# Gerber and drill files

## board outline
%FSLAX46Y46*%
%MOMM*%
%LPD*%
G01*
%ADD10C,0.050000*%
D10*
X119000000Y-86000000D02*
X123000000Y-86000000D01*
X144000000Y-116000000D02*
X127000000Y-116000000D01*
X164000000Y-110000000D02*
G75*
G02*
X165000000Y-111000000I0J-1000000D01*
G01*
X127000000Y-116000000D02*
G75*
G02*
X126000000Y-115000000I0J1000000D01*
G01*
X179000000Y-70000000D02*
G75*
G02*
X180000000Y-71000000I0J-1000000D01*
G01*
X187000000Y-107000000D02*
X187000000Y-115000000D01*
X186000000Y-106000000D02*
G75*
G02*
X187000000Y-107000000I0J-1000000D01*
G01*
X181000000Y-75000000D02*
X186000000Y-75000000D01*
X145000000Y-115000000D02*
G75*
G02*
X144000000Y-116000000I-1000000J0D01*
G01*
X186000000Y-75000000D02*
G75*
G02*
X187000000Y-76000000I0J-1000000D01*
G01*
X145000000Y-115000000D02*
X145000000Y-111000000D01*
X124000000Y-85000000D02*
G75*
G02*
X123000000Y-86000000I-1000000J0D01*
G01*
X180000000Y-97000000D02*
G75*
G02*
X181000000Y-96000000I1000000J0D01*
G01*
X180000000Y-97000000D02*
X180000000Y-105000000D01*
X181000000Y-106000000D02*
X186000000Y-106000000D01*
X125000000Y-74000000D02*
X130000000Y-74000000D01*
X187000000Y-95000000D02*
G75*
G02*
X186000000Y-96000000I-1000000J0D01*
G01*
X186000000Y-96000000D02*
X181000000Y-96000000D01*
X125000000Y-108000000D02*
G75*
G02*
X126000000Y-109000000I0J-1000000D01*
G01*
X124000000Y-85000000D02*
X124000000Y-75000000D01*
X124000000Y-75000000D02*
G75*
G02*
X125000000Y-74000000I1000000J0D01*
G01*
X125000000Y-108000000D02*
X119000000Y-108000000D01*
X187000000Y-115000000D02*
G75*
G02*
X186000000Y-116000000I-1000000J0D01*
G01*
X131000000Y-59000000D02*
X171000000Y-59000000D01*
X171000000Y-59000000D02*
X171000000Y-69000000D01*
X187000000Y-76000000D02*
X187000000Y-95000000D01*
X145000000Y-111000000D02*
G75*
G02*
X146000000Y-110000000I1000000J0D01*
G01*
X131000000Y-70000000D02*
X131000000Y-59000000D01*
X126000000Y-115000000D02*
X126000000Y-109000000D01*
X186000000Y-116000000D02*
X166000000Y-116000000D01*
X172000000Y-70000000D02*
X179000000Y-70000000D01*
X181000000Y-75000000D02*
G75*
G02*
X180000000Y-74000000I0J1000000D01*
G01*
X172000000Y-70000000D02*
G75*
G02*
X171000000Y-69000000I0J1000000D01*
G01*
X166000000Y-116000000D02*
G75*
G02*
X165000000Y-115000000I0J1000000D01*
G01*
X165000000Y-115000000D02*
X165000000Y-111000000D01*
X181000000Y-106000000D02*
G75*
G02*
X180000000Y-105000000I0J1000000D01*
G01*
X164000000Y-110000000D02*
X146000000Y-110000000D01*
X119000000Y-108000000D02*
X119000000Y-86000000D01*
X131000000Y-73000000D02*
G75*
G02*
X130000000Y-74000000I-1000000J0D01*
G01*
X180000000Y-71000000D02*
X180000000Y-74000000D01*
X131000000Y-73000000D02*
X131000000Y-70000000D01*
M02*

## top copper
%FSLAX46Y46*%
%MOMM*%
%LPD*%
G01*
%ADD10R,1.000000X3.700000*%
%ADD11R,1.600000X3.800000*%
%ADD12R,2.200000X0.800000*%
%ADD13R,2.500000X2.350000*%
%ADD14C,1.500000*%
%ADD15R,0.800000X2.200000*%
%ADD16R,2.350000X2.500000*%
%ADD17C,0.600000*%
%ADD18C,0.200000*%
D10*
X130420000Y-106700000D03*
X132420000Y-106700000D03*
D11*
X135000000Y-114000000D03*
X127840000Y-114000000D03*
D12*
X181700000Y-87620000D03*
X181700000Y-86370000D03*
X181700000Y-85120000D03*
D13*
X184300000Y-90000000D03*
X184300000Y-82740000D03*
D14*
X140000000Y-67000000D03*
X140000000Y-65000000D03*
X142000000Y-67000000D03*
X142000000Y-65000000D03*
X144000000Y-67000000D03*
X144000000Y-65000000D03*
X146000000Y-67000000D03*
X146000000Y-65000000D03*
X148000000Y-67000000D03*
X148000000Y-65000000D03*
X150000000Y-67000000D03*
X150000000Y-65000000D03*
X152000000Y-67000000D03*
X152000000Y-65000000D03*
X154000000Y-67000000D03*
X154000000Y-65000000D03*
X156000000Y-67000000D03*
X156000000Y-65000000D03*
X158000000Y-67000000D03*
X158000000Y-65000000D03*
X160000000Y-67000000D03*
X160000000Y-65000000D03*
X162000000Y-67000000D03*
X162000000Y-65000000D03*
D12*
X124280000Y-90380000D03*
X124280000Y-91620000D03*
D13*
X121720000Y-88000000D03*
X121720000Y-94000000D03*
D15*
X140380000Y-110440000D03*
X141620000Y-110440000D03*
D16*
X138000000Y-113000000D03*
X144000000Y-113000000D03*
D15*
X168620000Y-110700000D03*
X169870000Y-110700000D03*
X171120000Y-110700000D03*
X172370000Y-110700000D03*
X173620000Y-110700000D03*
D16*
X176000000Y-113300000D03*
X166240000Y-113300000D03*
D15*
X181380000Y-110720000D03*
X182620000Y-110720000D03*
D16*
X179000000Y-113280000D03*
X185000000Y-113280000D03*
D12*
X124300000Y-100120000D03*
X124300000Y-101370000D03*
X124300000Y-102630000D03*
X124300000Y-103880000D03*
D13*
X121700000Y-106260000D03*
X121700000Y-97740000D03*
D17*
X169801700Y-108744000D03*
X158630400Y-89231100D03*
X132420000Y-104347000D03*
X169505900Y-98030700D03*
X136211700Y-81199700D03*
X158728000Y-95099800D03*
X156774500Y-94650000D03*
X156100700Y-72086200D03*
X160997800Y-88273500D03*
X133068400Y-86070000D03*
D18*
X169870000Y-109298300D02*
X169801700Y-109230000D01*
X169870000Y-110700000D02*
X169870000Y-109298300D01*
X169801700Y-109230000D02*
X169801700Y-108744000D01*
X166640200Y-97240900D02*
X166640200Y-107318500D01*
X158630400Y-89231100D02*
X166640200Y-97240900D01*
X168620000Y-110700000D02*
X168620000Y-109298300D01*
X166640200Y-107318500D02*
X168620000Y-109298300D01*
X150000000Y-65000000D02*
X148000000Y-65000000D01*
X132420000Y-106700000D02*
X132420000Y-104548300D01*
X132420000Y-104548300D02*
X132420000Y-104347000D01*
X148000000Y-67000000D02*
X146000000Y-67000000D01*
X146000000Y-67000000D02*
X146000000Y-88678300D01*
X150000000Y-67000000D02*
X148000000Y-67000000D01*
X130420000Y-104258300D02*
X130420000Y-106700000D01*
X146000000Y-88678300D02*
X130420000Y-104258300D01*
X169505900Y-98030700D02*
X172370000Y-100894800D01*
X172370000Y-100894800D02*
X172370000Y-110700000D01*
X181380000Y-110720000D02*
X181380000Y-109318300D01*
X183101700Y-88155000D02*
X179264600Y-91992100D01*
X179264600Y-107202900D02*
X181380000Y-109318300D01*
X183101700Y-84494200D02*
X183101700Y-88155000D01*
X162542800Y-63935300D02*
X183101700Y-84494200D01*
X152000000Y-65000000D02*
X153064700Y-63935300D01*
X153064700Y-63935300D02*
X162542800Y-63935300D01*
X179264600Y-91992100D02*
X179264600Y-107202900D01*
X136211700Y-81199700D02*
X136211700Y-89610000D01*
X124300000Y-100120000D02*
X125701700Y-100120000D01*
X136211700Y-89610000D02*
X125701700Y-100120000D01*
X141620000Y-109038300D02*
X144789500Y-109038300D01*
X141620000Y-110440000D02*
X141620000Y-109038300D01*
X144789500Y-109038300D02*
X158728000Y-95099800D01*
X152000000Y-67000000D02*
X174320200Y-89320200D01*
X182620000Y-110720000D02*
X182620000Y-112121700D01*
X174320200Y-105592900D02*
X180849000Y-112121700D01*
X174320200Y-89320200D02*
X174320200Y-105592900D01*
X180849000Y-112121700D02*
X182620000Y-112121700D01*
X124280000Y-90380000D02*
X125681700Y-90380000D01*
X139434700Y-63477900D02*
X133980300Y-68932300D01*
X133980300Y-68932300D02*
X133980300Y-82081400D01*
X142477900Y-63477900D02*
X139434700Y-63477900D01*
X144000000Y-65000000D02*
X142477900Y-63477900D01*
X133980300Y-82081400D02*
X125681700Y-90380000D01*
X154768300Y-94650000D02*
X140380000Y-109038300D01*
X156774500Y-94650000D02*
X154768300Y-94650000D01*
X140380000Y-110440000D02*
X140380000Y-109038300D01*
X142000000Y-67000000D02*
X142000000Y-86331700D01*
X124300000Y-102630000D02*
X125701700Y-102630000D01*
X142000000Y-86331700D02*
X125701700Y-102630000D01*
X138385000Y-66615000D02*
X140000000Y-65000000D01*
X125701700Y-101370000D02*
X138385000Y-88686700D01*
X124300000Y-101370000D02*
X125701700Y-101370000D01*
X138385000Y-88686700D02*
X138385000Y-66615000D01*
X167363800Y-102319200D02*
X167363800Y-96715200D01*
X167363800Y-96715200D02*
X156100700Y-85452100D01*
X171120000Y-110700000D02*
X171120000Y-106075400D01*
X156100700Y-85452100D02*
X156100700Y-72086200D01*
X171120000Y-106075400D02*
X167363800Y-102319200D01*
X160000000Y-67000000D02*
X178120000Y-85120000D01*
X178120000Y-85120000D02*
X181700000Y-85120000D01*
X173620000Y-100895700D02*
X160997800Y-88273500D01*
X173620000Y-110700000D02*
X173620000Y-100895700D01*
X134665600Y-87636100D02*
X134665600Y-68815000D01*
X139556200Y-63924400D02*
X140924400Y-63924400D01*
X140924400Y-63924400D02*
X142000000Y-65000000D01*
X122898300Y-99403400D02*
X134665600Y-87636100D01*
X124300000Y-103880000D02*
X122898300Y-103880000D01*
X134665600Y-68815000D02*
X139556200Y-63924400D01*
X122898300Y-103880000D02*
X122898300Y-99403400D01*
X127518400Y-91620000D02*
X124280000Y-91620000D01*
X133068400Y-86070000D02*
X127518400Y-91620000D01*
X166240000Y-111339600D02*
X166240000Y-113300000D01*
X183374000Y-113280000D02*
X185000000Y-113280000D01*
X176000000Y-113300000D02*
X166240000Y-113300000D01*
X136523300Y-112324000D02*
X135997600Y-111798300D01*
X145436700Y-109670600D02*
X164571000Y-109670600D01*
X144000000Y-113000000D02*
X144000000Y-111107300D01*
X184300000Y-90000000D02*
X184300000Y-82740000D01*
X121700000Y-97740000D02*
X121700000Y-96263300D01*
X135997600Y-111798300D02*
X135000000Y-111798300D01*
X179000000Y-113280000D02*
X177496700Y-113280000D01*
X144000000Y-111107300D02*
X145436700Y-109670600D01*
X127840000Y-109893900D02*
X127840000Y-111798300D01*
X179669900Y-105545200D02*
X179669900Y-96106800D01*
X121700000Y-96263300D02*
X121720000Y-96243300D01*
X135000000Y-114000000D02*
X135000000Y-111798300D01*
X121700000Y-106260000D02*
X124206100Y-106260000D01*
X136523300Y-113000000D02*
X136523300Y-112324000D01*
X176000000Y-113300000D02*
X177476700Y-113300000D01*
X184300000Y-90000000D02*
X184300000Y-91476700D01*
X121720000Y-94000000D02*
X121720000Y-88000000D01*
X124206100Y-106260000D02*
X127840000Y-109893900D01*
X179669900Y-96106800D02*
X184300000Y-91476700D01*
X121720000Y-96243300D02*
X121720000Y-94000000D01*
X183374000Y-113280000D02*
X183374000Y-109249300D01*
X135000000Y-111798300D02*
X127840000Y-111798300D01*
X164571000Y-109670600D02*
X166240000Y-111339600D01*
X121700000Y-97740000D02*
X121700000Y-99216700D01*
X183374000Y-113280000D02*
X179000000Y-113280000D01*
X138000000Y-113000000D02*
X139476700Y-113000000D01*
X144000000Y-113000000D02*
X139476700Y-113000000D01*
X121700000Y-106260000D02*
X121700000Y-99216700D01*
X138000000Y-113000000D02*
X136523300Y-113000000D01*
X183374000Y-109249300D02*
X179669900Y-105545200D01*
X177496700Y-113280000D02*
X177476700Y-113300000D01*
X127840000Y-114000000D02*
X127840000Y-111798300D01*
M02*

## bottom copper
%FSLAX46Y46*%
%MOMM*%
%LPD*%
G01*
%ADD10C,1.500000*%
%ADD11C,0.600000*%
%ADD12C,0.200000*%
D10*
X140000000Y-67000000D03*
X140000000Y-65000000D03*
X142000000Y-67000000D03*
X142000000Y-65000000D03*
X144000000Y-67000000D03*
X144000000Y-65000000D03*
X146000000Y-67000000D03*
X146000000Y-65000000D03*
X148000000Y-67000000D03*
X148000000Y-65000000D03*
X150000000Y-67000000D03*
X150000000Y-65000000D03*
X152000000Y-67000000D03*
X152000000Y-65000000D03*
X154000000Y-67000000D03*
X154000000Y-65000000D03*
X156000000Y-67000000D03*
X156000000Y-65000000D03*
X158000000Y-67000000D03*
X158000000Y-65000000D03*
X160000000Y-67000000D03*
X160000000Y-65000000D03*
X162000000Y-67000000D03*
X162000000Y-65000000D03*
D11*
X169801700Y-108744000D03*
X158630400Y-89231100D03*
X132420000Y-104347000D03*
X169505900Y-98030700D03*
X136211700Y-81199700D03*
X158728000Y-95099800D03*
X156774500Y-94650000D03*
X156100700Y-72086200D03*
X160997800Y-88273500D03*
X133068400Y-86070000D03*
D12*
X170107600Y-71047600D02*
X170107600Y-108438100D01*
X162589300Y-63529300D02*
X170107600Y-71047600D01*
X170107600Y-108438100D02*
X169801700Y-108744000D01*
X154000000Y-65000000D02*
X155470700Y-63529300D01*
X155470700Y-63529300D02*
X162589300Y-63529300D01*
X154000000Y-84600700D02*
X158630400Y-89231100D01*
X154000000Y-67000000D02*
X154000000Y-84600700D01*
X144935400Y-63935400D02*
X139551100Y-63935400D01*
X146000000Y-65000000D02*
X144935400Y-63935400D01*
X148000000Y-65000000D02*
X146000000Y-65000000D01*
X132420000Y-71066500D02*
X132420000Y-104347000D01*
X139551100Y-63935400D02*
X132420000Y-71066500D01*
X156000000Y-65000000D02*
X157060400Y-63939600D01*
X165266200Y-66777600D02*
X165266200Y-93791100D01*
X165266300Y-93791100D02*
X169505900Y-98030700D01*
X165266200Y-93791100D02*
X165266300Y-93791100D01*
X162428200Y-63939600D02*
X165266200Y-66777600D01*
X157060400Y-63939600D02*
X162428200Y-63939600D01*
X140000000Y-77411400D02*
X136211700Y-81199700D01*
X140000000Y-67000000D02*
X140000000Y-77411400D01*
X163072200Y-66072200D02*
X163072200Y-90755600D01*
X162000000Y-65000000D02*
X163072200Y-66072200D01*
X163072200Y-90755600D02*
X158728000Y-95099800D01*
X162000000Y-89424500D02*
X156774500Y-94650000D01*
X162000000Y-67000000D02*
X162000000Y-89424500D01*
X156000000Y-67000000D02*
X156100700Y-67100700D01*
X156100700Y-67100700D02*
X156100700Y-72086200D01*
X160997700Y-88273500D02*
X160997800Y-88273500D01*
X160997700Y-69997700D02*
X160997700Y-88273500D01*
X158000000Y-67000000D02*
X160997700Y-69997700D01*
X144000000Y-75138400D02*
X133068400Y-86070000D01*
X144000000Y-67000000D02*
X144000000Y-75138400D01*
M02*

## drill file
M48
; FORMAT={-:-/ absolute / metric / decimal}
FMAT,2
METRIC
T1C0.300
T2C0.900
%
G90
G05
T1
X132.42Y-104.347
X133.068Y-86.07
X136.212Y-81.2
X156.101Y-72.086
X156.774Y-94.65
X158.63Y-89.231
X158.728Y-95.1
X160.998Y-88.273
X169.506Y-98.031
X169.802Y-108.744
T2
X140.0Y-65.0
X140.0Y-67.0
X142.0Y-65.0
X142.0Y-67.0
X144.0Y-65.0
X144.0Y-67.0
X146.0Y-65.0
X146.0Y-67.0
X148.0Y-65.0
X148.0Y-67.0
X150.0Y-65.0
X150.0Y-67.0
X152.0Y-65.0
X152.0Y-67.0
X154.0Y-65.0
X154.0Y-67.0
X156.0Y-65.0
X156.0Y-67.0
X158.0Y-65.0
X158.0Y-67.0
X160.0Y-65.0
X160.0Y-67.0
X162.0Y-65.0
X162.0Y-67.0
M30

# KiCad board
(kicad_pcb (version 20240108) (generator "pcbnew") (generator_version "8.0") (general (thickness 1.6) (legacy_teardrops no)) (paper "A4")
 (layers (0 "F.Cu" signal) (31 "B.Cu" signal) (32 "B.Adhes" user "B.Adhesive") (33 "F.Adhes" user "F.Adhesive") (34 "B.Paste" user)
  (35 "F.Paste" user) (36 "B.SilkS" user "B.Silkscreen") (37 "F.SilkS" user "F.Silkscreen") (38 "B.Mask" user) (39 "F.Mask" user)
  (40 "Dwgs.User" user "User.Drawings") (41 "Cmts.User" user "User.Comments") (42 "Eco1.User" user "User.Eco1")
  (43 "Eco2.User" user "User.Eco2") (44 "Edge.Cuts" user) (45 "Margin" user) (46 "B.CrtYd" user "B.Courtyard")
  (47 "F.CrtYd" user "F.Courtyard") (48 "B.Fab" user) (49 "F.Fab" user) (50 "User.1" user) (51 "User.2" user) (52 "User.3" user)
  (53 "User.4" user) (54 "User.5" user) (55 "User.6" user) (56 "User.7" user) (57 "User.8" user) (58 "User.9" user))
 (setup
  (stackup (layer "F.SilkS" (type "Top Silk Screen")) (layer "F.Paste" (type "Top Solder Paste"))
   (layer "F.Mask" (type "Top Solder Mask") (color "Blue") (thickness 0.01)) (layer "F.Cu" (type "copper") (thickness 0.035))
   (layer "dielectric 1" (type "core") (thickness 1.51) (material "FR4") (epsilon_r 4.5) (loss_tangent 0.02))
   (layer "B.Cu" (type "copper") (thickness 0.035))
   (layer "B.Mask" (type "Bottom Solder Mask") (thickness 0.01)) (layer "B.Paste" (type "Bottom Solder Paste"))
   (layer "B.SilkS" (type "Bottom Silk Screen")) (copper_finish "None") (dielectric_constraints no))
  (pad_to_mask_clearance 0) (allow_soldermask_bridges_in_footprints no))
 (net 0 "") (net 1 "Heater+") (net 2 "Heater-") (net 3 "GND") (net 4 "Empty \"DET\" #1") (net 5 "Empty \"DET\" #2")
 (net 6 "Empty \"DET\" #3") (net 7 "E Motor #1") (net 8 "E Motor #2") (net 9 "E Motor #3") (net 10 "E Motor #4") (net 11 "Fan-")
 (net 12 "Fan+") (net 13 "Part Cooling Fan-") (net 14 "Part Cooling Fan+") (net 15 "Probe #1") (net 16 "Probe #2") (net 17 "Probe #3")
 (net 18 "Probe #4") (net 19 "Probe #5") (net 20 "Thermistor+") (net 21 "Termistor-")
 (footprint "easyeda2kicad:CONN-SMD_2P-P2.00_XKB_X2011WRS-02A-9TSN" (layer "F.Cu") (at 131.42 110.35)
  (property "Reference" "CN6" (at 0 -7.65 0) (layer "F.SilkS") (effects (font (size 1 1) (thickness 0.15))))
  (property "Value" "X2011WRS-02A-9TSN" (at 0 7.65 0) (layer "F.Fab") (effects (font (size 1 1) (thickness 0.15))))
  (pad "1" smd rect (at -1 -3.65) (size 1 3.7) (layers "F.Cu" "F.Paste" "F.Mask") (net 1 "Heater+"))
  (pad "2" smd rect (at 1 -3.65) (size 1 3.7) (layers "F.Cu" "F.Paste" "F.Mask") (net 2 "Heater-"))
  (pad "3" smd rect (at 3.58 3.65) (size 1.6 3.8) (layers "F.Cu" "F.Paste" "F.Mask") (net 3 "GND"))
  (pad "4" smd rect (at -3.58 3.65) (size 1.6 3.8) (layers "F.Cu" "F.Paste" "F.Mask") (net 3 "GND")))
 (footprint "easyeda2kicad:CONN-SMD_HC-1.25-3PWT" (layer "F.Cu") (at 183 86.37 90)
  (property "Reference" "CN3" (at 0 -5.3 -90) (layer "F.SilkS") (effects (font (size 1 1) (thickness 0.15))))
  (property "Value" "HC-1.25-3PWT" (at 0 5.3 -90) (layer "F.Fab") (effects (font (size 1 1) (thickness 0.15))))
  (pad "1" smd rect (at -1.25 -1.3 90) (size 0.8 2.2) (layers "F.Cu" "F.Paste" "F.Mask") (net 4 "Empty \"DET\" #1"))
  (pad "2" smd rect (at 0 -1.3 90) (size 0.8 2.2) (layers "F.Cu" "F.Paste" "F.Mask") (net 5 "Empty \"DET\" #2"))
  (pad "3" smd rect (at 1.25 -1.3 90) (size 0.8 2.2) (layers "F.Cu" "F.Paste" "F.Mask") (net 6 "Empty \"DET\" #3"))
  (pad "4" smd rect (at -3.63 1.3 90) (size 2.35 2.5) (layers "F.Cu" "F.Paste" "F.Mask") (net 3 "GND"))
  (pad "5" smd rect (at 3.63 1.3 90) (size 2.35 2.5) (layers "F.Cu" "F.Paste" "F.Mask") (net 3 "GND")))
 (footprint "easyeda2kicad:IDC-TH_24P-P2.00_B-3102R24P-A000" (layer "F.Cu") (at 151 66 180)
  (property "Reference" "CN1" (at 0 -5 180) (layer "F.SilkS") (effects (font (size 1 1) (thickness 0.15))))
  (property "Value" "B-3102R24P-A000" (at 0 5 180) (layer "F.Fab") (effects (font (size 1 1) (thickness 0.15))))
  (pad "1" thru_hole circle (at 11 -1 90) (size 1.5 1.5) (drill 0.900024) (layers "*.Cu" "*.Mask") (remove_unused_layers no)
   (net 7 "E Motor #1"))
  (pad "2" thru_hole circle (at 11 1 90) (size 1.5 1.5) (drill 0.900024) (layers "*.Cu" "*.Mask") (remove_unused_layers no)
   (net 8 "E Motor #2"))
  (pad "3" thru_hole circle (at 9 -1 90) (size 1.5 1.5) (drill 0.900024) (layers "*.Cu" "*.Mask") (remove_unused_layers no)
   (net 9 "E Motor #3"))
  (pad "4" thru_hole circle (at 9 1 90) (size 1.5 1.5) (drill 0.900024) (layers "*.Cu" "*.Mask") (remove_unused_layers no)
   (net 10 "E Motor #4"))
  (pad "5" thru_hole circle (at 7 -1 90) (size 1.5 1.5) (drill 0.900024) (layers "*.Cu" "*.Mask") (remove_unused_layers no) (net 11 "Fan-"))
  (pad "6" thru_hole circle (at 7 1 90) (size 1.5 1.5) (drill 0.900024) (layers "*.Cu" "*.Mask") (remove_unused_layers no) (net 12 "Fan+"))
  (pad "7" thru_hole circle (at 5 -1 90) (size 1.5 1.5) (drill 0.900024) (layers "*.Cu" "*.Mask") (remove_unused_layers no)
   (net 1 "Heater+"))
  (pad "8" thru_hole circle (at 5 1 90) (size 1.5 1.5) (drill 0.900024) (layers "*.Cu" "*.Mask") (remove_unused_layers no) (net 2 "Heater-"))
  (pad "9" thru_hole circle (at 3 -1 90) (size 1.5 1.5) (drill 0.900024) (layers "*.Cu" "*.Mask") (remove_unused_layers no)
   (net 1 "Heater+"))
  (pad "10" thru_hole circle (at 3 1 90) (size 1.5 1.5) (drill 0.900024) (layers "*.Cu" "*.Mask") (remove_unused_layers no)
   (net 2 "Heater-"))
  (pad "11" thru_hole circle (at 1 -1 90) (size 1.5 1.5) (drill 0.900024) (layers "*.Cu" "*.Mask") (remove_unused_layers no)
   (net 1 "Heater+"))
  (pad "12" thru_hole circle (at 1 1 90) (size 1.5 1.5) (drill 0.900024) (layers "*.Cu" "*.Mask") (remove_unused_layers no)
   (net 2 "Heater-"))
  (pad "13" thru_hole circle (at -1 -1 90) (size 1.5 1.5) (drill 0.900024) (layers "*.Cu" "*.Mask") (remove_unused_layers no)
   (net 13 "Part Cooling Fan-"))
  (pad "14" thru_hole circle (at -1 1 90) (size 1.5 1.5) (drill 0.900024) (layers "*.Cu" "*.Mask") (remove_unused_layers no)
   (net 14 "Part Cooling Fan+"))
  (pad "15" thru_hole circle (at -3 -1 90) (size 1.5 1.5) (drill 0.900024) (layers "*.Cu" "*.Mask") (remove_unused_layers no)
   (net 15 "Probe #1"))
  (pad "16" thru_hole circle (at -3 1 90) (size 1.5 1.5) (drill 0.900024) (layers "*.Cu" "*.Mask") (remove_unused_layers no)
   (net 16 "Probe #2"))
  (pad "17" thru_hole circle (at -5 -1 90) (size 1.5 1.5) (drill 0.900024) (layers "*.Cu" "*.Mask") (remove_unused_layers no)
   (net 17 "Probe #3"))
  (pad "18" thru_hole circle (at -5 1 90) (size 1.5 1.5) (drill 0.900024) (layers "*.Cu" "*.Mask") (remove_unused_layers no)
   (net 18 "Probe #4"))
  (pad "19" thru_hole circle (at -7 -1 90) (size 1.5 1.5) (drill 0.900024) (layers "*.Cu" "*.Mask") (remove_unused_layers no)
   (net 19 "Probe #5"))
  (pad "20" thru_hole circle (at -7 1 90) (size 1.5 1.5) (drill 0.900024) (layers "*.Cu" "*.Mask") (remove_unused_layers no)
   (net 4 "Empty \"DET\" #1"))
  (pad "21" thru_hole circle (at -9 -1 90) (size 1.5 1.5) (drill 0.900024) (layers "*.Cu" "*.Mask") (remove_unused_layers no)
   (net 6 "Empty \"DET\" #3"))
  (pad "22" thru_hole circle (at -9 1 90) (size 1.5 1.5) (drill 0.900024) (layers "*.Cu" "*.Mask") (remove_unused_layers no)
   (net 5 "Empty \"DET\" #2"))
  (pad "23" thru_hole circle (at -11 -1 90) (size 1.5 1.5) (drill 0.900024) (layers "*.Cu" "*.Mask") (remove_unused_layers no)
   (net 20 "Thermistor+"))
  (pad "24" thru_hole circle (at -11 1 90) (size 1.5 1.5) (drill 0.900024) (layers "*.Cu" "*.Mask") (remove_unused_layers no)
   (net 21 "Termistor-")))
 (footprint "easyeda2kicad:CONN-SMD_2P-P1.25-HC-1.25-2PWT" (layer "F.Cu") (at 123 91 -90)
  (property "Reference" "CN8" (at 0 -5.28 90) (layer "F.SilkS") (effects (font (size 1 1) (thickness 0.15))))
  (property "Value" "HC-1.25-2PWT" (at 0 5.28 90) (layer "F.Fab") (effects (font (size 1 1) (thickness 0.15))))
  (pad "1" smd rect (at -0.62 -1.28 270) (size 0.8 2.2) (layers "F.Cu" "F.Paste" "F.Mask") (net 12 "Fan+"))
  (pad "2" smd rect (at 0.62 -1.28 270) (size 0.8 2.2) (layers "F.Cu" "F.Paste" "F.Mask") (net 11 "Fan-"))
  (pad "3" smd rect (at -3 1.28 180) (size 2.5 2.35) (layers "F.Cu" "F.Paste" "F.Mask") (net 3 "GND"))
  (pad "4" smd rect (at 3 1.28) (size 2.5 2.35) (layers "F.Cu" "F.Paste" "F.Mask") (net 3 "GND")))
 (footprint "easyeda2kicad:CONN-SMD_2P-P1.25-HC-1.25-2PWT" (layer "F.Cu") (at 141 111.72)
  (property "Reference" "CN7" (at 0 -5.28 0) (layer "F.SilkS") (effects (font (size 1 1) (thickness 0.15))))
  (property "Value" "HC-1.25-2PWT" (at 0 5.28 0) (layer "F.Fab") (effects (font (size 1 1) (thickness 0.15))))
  (pad "1" smd rect (at -0.62 -1.28) (size 0.8 2.2) (layers "F.Cu" "F.Paste" "F.Mask") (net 20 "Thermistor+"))
  (pad "2" smd rect (at 0.62 -1.28) (size 0.8 2.2) (layers "F.Cu" "F.Paste" "F.Mask") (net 21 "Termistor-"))
  (pad "3" smd rect (at -3 1.28 270) (size 2.5 2.35) (layers "F.Cu" "F.Paste" "F.Mask") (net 3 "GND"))
  (pad "4" smd rect (at 3 1.28 90) (size 2.5 2.35) (layers "F.Cu" "F.Paste" "F.Mask") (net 3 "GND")))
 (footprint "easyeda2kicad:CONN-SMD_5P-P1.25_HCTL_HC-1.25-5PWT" (layer "F.Cu") (at 171.12 112)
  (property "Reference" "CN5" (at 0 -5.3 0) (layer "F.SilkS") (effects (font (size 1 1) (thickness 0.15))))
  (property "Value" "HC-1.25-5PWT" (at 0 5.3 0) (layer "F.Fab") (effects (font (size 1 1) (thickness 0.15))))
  (pad "1" smd rect (at -2.5 -1.3) (size 0.8 2.2) (layers "F.Cu" "F.Paste" "F.Mask") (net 15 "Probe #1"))
  (pad "2" smd rect (at -1.25 -1.3) (size 0.8 2.2) (layers "F.Cu" "F.Paste" "F.Mask") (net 16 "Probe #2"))
  (pad "3" smd rect (at 0 -1.3) (size 0.8 2.2) (layers "F.Cu" "F.Paste" "F.Mask") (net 17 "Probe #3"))
  (pad "4" smd rect (at 1.25 -1.3) (size 0.8 2.2) (layers "F.Cu" "F.Paste" "F.Mask") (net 18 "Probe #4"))
  (pad "5" smd rect (at 2.5 -1.3) (size 0.8 2.2) (layers "F.Cu" "F.Paste" "F.Mask") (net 19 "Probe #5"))
  (pad "6" smd rect (at 4.88 1.3) (size 2.35 2.5) (layers "F.Cu" "F.Paste" "F.Mask") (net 3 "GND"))
  (pad "7" smd rect (at -4.88 1.3) (size 2.35 2.5) (layers "F.Cu" "F.Paste" "F.Mask") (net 3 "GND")))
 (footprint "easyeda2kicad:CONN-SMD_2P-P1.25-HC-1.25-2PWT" (layer "F.Cu") (at 182 112)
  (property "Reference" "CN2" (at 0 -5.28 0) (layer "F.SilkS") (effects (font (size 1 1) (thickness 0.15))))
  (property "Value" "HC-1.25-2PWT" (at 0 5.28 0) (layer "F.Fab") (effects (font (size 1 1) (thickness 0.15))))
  (pad "1" smd rect (at -0.62 -1.28) (size 0.8 2.2) (layers "F.Cu" "F.Paste" "F.Mask") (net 14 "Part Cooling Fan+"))
  (pad "2" smd rect (at 0.62 -1.28) (size 0.8 2.2) (layers "F.Cu" "F.Paste" "F.Mask") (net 13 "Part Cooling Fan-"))
  (pad "3" smd rect (at -3 1.28 270) (size 2.5 2.35) (layers "F.Cu" "F.Paste" "F.Mask") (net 3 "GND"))
  (pad "4" smd rect (at 3 1.28 90) (size 2.5 2.35) (layers "F.Cu" "F.Paste" "F.Mask") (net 3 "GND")))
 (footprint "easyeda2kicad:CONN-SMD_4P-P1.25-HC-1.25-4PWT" (layer "F.Cu") (at 123 102 -90)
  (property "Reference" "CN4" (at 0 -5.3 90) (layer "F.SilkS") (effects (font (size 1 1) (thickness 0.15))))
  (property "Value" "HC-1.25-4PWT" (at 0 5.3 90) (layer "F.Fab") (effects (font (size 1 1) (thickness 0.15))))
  (pad "1" smd rect (at -1.88 -1.3) (size 2.2 0.8) (layers "F.Cu" "F.Paste" "F.Mask") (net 7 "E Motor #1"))
  (pad "2" smd rect (at -0.63 -1.3) (size 2.2 0.8) (layers "F.Cu" "F.Paste" "F.Mask") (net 8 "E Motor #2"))
  (pad "3" smd rect (at 0.63 -1.3) (size 2.2 0.8) (layers "F.Cu" "F.Paste" "F.Mask") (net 9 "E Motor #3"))
  (pad "4" smd rect (at 1.88 -1.3) (size 2.2 0.8) (layers "F.Cu" "F.Paste" "F.Mask") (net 10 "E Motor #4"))
  (pad "5" smd rect (at 4.26 1.3 90) (size 2.35 2.5) (layers "F.Cu" "F.Paste" "F.Mask") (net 3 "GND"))
  (pad "6" smd rect (at -4.26 1.3 90) (size 2.35 2.5) (layers "F.Cu" "F.Paste" "F.Mask") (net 3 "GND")))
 (gr_line (start 119 86) (end 123 86) (stroke (width 0.05) (type default)) (layer "Edge.Cuts"))
 (gr_line (start 144 116) (end 127 116) (stroke (width 0.05) (type default)) (layer "Edge.Cuts"))
 (gr_arc (start 164 110) (mid 164.707107 110.292893) (end 165 111) (stroke (width 0.05) (type default)) (layer "Edge.Cuts"))
 (gr_arc (start 127 116) (mid 126.292893 115.707107) (end 126 115) (stroke (width 0.05) (type default)) (layer "Edge.Cuts"))
 (gr_arc (start 179 70) (mid 179.707107 70.292893) (end 180 71) (stroke (width 0.05) (type default)) (layer "Edge.Cuts"))
 (gr_line (start 187 107) (end 187 115) (stroke (width 0.05) (type default)) (layer "Edge.Cuts"))
 (gr_arc (start 186 106) (mid 186.707107 106.292893) (end 187 107) (stroke (width 0.05) (type default)) (layer "Edge.Cuts"))
 (gr_line (start 181 75) (end 186 75) (stroke (width 0.05) (type default)) (layer "Edge.Cuts"))
 (gr_arc (start 145 115) (mid 144.707107 115.707107) (end 144 116) (stroke (width 0.05) (type default)) (layer "Edge.Cuts"))
 (gr_arc (start 186 75) (mid 186.707107 75.292893) (end 187 76) (stroke (width 0.05) (type default)) (layer "Edge.Cuts"))
 (gr_line (start 145 115) (end 145 111) (stroke (width 0.05) (type default)) (layer "Edge.Cuts"))
 (gr_arc (start 124 85) (mid 123.707107 85.707107) (end 123 86) (stroke (width 0.05) (type default)) (layer "Edge.Cuts"))
 (gr_arc (start 180 97) (mid 180.292893 96.292893) (end 181 96) (stroke (width 0.05) (type default)) (layer "Edge.Cuts"))
 (gr_line (start 180 97) (end 180 105) (stroke (width 0.05) (type default)) (layer "Edge.Cuts"))
 (gr_line (start 181 106) (end 186 106) (stroke (width 0.05) (type default)) (layer "Edge.Cuts"))
 (gr_line (start 125 74) (end 130 74) (stroke (width 0.05) (type default)) (layer "Edge.Cuts"))
 (gr_arc (start 187 95) (mid 186.707107 95.707107) (end 186 96) (stroke (width 0.05) (type default)) (layer "Edge.Cuts"))
 (gr_line (start 186 96) (end 181 96) (stroke (width 0.05) (type default)) (layer "Edge.Cuts"))
 (gr_arc (start 125 108) (mid 125.707107 108.292893) (end 126 109) (stroke (width 0.05) (type default)) (layer "Edge.Cuts"))
 (gr_line (start 124 85) (end 124 75) (stroke (width 0.05) (type default)) (layer "Edge.Cuts"))
 (gr_arc (start 124 75) (mid 124.292893 74.292893) (end 125 74) (stroke (width 0.05) (type default)) (layer "Edge.Cuts"))
 (gr_line (start 125 108) (end 119 108) (stroke (width 0.05) (type default)) (layer "Edge.Cuts"))
 (gr_arc (start 187 115) (mid 186.707107 115.707107) (end 186 116) (stroke (width 0.05) (type default)) (layer "Edge.Cuts"))
 (gr_line (start 131 59) (end 171 59) (stroke (width 0.05) (type default)) (layer "Edge.Cuts"))
 (gr_line (start 171 59) (end 171 69) (stroke (width 0.05) (type default)) (layer "Edge.Cuts"))
 (gr_line (start 187 76) (end 187 95) (stroke (width 0.05) (type default)) (layer "Edge.Cuts"))
 (gr_arc (start 145 111) (mid 145.292893 110.292893) (end 146 110) (stroke (width 0.05) (type default)) (layer "Edge.Cuts"))
 (gr_line (start 131 70) (end 131 59) (stroke (width 0.05) (type default)) (layer "Edge.Cuts"))
 (gr_line (start 126 115) (end 126 109) (stroke (width 0.05) (type default)) (layer "Edge.Cuts"))
 (gr_line (start 186 116) (end 166 116) (stroke (width 0.05) (type default)) (layer "Edge.Cuts"))
 (gr_line (start 172 70) (end 179 70) (stroke (width 0.05) (type default)) (layer "Edge.Cuts"))
 (gr_arc (start 181 75) (mid 180.292893 74.707107) (end 180 74) (stroke (width 0.05) (type default)) (layer "Edge.Cuts"))
 (gr_arc (start 172 70) (mid 171.292893 69.707107) (end 171 69) (stroke (width 0.05) (type default)) (layer "Edge.Cuts"))
 (gr_arc (start 166 116) (mid 165.292893 115.707107) (end 165 115) (stroke (width 0.05) (type default)) (layer "Edge.Cuts"))
 (gr_line (start 165 115) (end 165 111) (stroke (width 0.05) (type default)) (layer "Edge.Cuts"))
 (gr_arc (start 181 106) (mid 180.292893 105.707107) (end 180 105) (stroke (width 0.05) (type default)) (layer "Edge.Cuts"))
 (gr_line (start 164 110) (end 146 110) (stroke (width 0.05) (type default)) (layer "Edge.Cuts"))
 (gr_line (start 119 108) (end 119 86) (stroke (width 0.05) (type default)) (layer "Edge.Cuts"))
 (gr_arc (start 131 73) (mid 130.707107 73.707107) (end 130 74) (stroke (width 0.05) (type default)) (layer "Edge.Cuts"))
 (gr_line (start 180 71) (end 180 74) (stroke (width 0.05) (type default)) (layer "Edge.Cuts"))
 (gr_line (start 131 73) (end 131 70) (stroke (width 0.05) (type default)) (layer "Edge.Cuts"))
 (segment (start 169.87 109.2983) (end 169.8017 109.23) (width 0.2) (layer "F.Cu") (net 16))
 (segment (start 169.87 110.7) (end 169.87 109.2983) (width 0.2) (layer "F.Cu") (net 16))
 (segment (start 169.8017 109.23) (end 169.8017 108.744) (width 0.2) (layer "F.Cu") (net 16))
 (via (at 169.8017 108.744) (size 0.6) (drill 0.3) (layers "F.Cu" "B.Cu") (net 16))
 (segment (start 170.1076 71.0476) (end 170.1076 108.4381) (width 0.2) (layer "B.Cu") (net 16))
 (segment (start 162.5893 63.5293) (end 170.1076 71.0476) (width 0.2) (layer "B.Cu") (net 16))
 (segment (start 170.1076 108.4381) (end 169.8017 108.744) (width 0.2) (layer "B.Cu") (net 16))
 (segment (start 154 65) (end 155.4707 63.5293) (width 0.2) (layer "B.Cu") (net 16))
 (segment (start 155.4707 63.5293) (end 162.5893 63.5293) (width 0.2) (layer "B.Cu") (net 16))
 (segment (start 166.6402 97.2409) (end 166.6402 107.3185) (width 0.2) (layer "F.Cu") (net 15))
 (segment (start 158.6304 89.2311) (end 166.6402 97.2409) (width 0.2) (layer "F.Cu") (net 15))
 (segment (start 168.62 110.7) (end 168.62 109.2983) (width 0.2) (layer "F.Cu") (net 15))
 (segment (start 166.6402 107.3185) (end 168.62 109.2983) (width 0.2) (layer "F.Cu") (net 15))
 (via (at 158.6304 89.2311) (size 0.6) (drill 0.3) (layers "F.Cu" "B.Cu") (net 15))
 (segment (start 154 84.6007) (end 158.6304 89.2311) (width 0.2) (layer "B.Cu") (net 15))
 (segment (start 154 67) (end 154 84.6007) (width 0.2) (layer "B.Cu") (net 15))
 (segment (start 150 65) (end 148 65) (width 0.2) (layer "F.Cu") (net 2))
 (segment (start 132.42 106.7) (end 132.42 104.5483) (width 0.2) (layer "F.Cu") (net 2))
 (segment (start 132.42 104.5483) (end 132.42 104.347) (width 0.2) (layer "F.Cu") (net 2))
 (via (at 132.42 104.347) (size 0.6) (drill 0.3) (layers "F.Cu" "B.Cu") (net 2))
 (segment (start 144.9354 63.9354) (end 139.5511 63.9354) (width 0.2) (layer "B.Cu") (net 2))
 (segment (start 146 65) (end 144.9354 63.9354) (width 0.2) (layer "B.Cu") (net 2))
 (segment (start 148 65) (end 146 65) (width 0.2) (layer "B.Cu") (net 2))
 (segment (start 132.42 71.0665) (end 132.42 104.347) (width 0.2) (layer "B.Cu") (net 2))
 (segment (start 139.5511 63.9354) (end 132.42 71.0665) (width 0.2) (layer "B.Cu") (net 2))
 (segment (start 148 67) (end 146 67) (width 0.2) (layer "F.Cu") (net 1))
 (segment (start 146 67) (end 146 88.6783) (width 0.2) (layer "F.Cu") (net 1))
 (segment (start 150 67) (end 148 67) (width 0.2) (layer "F.Cu") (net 1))
 (segment (start 130.42 104.2583) (end 130.42 106.7) (width 0.2) (layer "F.Cu") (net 1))
 (segment (start 146 88.6783) (end 130.42 104.2583) (width 0.2) (layer "F.Cu") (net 1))
 (segment (start 169.5059 98.0307) (end 172.37 100.8948) (width 0.2) (layer "F.Cu") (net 18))
 (segment (start 172.37 100.8948) (end 172.37 110.7) (width 0.2) (layer "F.Cu") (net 18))
 (via (at 169.5059 98.0307) (size 0.6) (drill 0.3) (layers "F.Cu" "B.Cu") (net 18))
 (segment (start 156 65) (end 157.0604 63.9396) (width 0.2) (layer "B.Cu") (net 18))
 (segment (start 165.2662 66.7776) (end 165.2662 93.7911) (width 0.2) (layer "B.Cu") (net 18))
 (segment (start 165.2663 93.7911) (end 169.5059 98.0307) (width 0.2) (layer "B.Cu") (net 18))
 (segment (start 165.2662 93.7911) (end 165.2663 93.7911) (width 0.2) (layer "B.Cu") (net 18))
 (segment (start 162.4282 63.9396) (end 165.2662 66.7776) (width 0.2) (layer "B.Cu") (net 18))
 (segment (start 157.0604 63.9396) (end 162.4282 63.9396) (width 0.2) (layer "B.Cu") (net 18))
 (segment (start 181.38 110.72) (end 181.38 109.3183) (width 0.2) (layer "F.Cu") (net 14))
 (segment (start 183.1017 88.155) (end 179.2646 91.9921) (width 0.2) (layer "F.Cu") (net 14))
 (segment (start 179.2646 107.2029) (end 181.38 109.3183) (width 0.2) (layer "F.Cu") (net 14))
 (segment (start 183.1017 84.4942) (end 183.1017 88.155) (width 0.2) (layer "F.Cu") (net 14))
 (segment (start 162.5428 63.9353) (end 183.1017 84.4942) (width 0.2) (layer "F.Cu") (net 14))
 (segment (start 152 65) (end 153.0647 63.9353) (width 0.2) (layer "F.Cu") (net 14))
 (segment (start 153.0647 63.9353) (end 162.5428 63.9353) (width 0.2) (layer "F.Cu") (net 14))
 (segment (start 179.2646 91.9921) (end 179.2646 107.2029) (width 0.2) (layer "F.Cu") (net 14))
 (segment (start 136.2117 81.1997) (end 136.2117 89.61) (width 0.2) (layer "F.Cu") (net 7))
 (segment (start 124.3 100.12) (end 125.7017 100.12) (width 0.2) (layer "F.Cu") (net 7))
 (segment (start 136.2117 89.61) (end 125.7017 100.12) (width 0.2) (layer "F.Cu") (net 7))
 (via (at 136.2117 81.1997) (size 0.6) (drill 0.3) (layers "F.Cu" "B.Cu") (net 7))
 (segment (start 140 77.4114) (end 136.2117 81.1997) (width 0.2) (layer "B.Cu") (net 7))
 (segment (start 140 67) (end 140 77.4114) (width 0.2) (layer "B.Cu") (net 7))
 (segment (start 141.62 109.0383) (end 144.7895 109.0383) (width 0.2) (layer "F.Cu") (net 21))
 (segment (start 141.62 110.44) (end 141.62 109.0383) (width 0.2) (layer "F.Cu") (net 21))
 (segment (start 144.7895 109.0383) (end 158.728 95.0998) (width 0.2) (layer "F.Cu") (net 21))
 (via (at 158.728 95.0998) (size 0.6) (drill 0.3) (layers "F.Cu" "B.Cu") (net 21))
 (segment (start 163.0722 66.0722) (end 163.0722 90.7556) (width 0.2) (layer "B.Cu") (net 21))
 (segment (start 162 65) (end 163.0722 66.0722) (width 0.2) (layer "B.Cu") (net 21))
 (segment (start 163.0722 90.7556) (end 158.728 95.0998) (width 0.2) (layer "B.Cu") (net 21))
 (segment (start 152 67) (end 174.3202 89.3202) (width 0.2) (layer "F.Cu") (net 13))
 (segment (start 182.62 110.72) (end 182.62 112.1217) (width 0.2) (layer "F.Cu") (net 13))
 (segment (start 174.3202 105.5929) (end 180.849 112.1217) (width 0.2) (layer "F.Cu") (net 13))
 (segment (start 174.3202 89.3202) (end 174.3202 105.5929) (width 0.2) (layer "F.Cu") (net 13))
 (segment (start 180.849 112.1217) (end 182.62 112.1217) (width 0.2) (layer "F.Cu") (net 13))
 (segment (start 124.28 90.38) (end 125.6817 90.38) (width 0.2) (layer "F.Cu") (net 12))
 (segment (start 139.4347 63.4779) (end 133.9803 68.9323) (width 0.2) (layer "F.Cu") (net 12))
 (segment (start 133.9803 68.9323) (end 133.9803 82.0814) (width 0.2) (layer "F.Cu") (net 12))
 (segment (start 142.4779 63.4779) (end 139.4347 63.4779) (width 0.2) (layer "F.Cu") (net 12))
 (segment (start 144 65) (end 142.4779 63.4779) (width 0.2) (layer "F.Cu") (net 12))
 (segment (start 133.9803 82.0814) (end 125.6817 90.38) (width 0.2) (layer "F.Cu") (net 12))
 (segment (start 154.7683 94.65) (end 140.38 109.0383) (width 0.2) (layer "F.Cu") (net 20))
 (segment (start 156.7745 94.65) (end 154.7683 94.65) (width 0.2) (layer "F.Cu") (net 20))
 (segment (start 140.38 110.44) (end 140.38 109.0383) (width 0.2) (layer "F.Cu") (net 20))
 (via (at 156.7745 94.65) (size 0.6) (drill 0.3) (layers "F.Cu" "B.Cu") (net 20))
 (segment (start 162 89.4245) (end 156.7745 94.65) (width 0.2) (layer "B.Cu") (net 20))
 (segment (start 162 67) (end 162 89.4245) (width 0.2) (layer "B.Cu") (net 20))
 (segment (start 142 67) (end 142 86.3317) (width 0.2) (layer "F.Cu") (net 9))
 (segment (start 124.3 102.63) (end 125.7017 102.63) (width 0.2) (layer "F.Cu") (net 9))
 (segment (start 142 86.3317) (end 125.7017 102.63) (width 0.2) (layer "F.Cu") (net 9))
 (segment (start 138.385 66.615) (end 140 65) (width 0.2) (layer "F.Cu") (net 8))
 (segment (start 125.7017 101.37) (end 138.385 88.6867) (width 0.2) (layer "F.Cu") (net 8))
 (segment (start 124.3 101.37) (end 125.7017 101.37) (width 0.2) (layer "F.Cu") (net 8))
 (segment (start 138.385 88.6867) (end 138.385 66.615) (width 0.2) (layer "F.Cu") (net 8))
 (segment (start 167.3638 102.3192) (end 167.3638 96.7152) (width 0.2) (layer "F.Cu") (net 17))
 (segment (start 167.3638 96.7152) (end 156.1007 85.4521) (width 0.2) (layer "F.Cu") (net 17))
 (segment (start 171.12 110.7) (end 171.12 106.0754) (width 0.2) (layer "F.Cu") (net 17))
 (segment (start 156.1007 85.4521) (end 156.1007 72.0862) (width 0.2) (layer "F.Cu") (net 17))
 (segment (start 171.12 106.0754) (end 167.3638 102.3192) (width 0.2) (layer "F.Cu") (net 17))
 (via (at 156.1007 72.0862) (size 0.6) (drill 0.3) (layers "F.Cu" "B.Cu") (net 17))
 (segment (start 156 67) (end 156.1007 67.1007) (width 0.2) (layer "B.Cu") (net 17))
 (segment (start 156.1007 67.1007) (end 156.1007 72.0862) (width 0.2) (layer "B.Cu") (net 17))
 (segment (start 160 67) (end 178.12 85.12) (width 0.2) (layer "F.Cu") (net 6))
 (segment (start 178.12 85.12) (end 181.7 85.12) (width 0.2) (layer "F.Cu") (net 6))
 (segment (start 173.62 100.8957) (end 160.9978 88.2735) (width 0.2) (layer "F.Cu") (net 19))
 (segment (start 173.62 110.7) (end 173.62 100.8957) (width 0.2) (layer "F.Cu") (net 19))
 (via (at 160.9978 88.2735) (size 0.6) (drill 0.3) (layers "F.Cu" "B.Cu") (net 19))
 (segment (start 160.9977 88.2735) (end 160.9978 88.2735) (width 0.2) (layer "B.Cu") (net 19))
 (segment (start 160.9977 69.9977) (end 160.9977 88.2735) (width 0.2) (layer "B.Cu") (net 19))
 (segment (start 158 67) (end 160.9977 69.9977) (width 0.2) (layer "B.Cu") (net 19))
 (segment (start 134.6656 87.6361) (end 134.6656 68.815) (width 0.2) (layer "F.Cu") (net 10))
 (segment (start 139.5562 63.9244) (end 140.9244 63.9244) (width 0.2) (layer "F.Cu") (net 10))
 (segment (start 140.9244 63.9244) (end 142 65) (width 0.2) (layer "F.Cu") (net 10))
 (segment (start 122.8983 99.4034) (end 134.6656 87.6361) (width 0.2) (layer "F.Cu") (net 10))
 (segment (start 124.3 103.88) (end 122.8983 103.88) (width 0.2) (layer "F.Cu") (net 10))
 (segment (start 134.6656 68.815) (end 139.5562 63.9244) (width 0.2) (layer "F.Cu") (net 10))
 (segment (start 122.8983 103.88) (end 122.8983 99.4034) (width 0.2) (layer "F.Cu") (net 10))
 (segment (start 127.5184 91.62) (end 124.28 91.62) (width 0.2) (layer "F.Cu") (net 11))
 (segment (start 133.0684 86.07) (end 127.5184 91.62) (width 0.2) (layer "F.Cu") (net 11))
 (via (at 133.0684 86.07) (size 0.6) (drill 0.3) (layers "F.Cu" "B.Cu") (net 11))
 (segment (start 144 75.1384) (end 133.0684 86.07) (width 0.2) (layer "B.Cu") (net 11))
 (segment (start 144 67) (end 144 75.1384) (width 0.2) (layer "B.Cu") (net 11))
 (segment (start 166.24 111.3396) (end 166.24 113.3) (width 0.2) (layer "F.Cu") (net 3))
 (segment (start 183.374 113.28) (end 185 113.28) (width 0.2) (layer "F.Cu") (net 3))
 (segment (start 176 113.3) (end 166.24 113.3) (width 0.2) (layer "F.Cu") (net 3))
 (segment (start 136.5233 112.324) (end 135.9976 111.7983) (width 0.2) (layer "F.Cu") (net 3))
 (segment (start 145.4367 109.6706) (end 164.571 109.6706) (width 0.2) (layer "F.Cu") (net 3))
 (segment (start 144 113) (end 144 111.1073) (width 0.2) (layer "F.Cu") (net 3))
 (segment (start 184.3 90) (end 184.3 82.74) (width 0.2) (layer "F.Cu") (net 3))
 (segment (start 121.7 97.74) (end 121.7 96.2633) (width 0.2) (layer "F.Cu") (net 3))
 (segment (start 135.9976 111.7983) (end 135 111.7983) (width 0.2) (layer "F.Cu") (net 3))
 (segment (start 179 113.28) (end 177.4967 113.28) (width 0.2) (layer "F.Cu") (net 3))
 (segment (start 144 111.1073) (end 145.4367 109.6706) (width 0.2) (layer "F.Cu") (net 3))
 (segment (start 127.84 109.8939) (end 127.84 111.7983) (width 0.2) (layer "F.Cu") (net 3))
 (segment (start 179.6699 105.5452) (end 179.6699 96.1068) (width 0.2) (layer "F.Cu") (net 3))
 (segment (start 121.7 96.2633) (end 121.72 96.2433) (width 0.2) (layer "F.Cu") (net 3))
 (segment (start 135 114) (end 135 111.7983) (width 0.2) (layer "F.Cu") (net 3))
 (segment (start 121.7 106.26) (end 124.2061 106.26) (width 0.2) (layer "F.Cu") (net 3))
 (segment (start 136.5233 113) (end 136.5233 112.324) (width 0.2) (layer "F.Cu") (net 3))
 (segment (start 176 113.3) (end 177.4767 113.3) (width 0.2) (layer "F.Cu") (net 3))
 (segment (start 184.3 90) (end 184.3 91.4767) (width 0.2) (layer "F.Cu") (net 3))
 (segment (start 121.72 94) (end 121.72 88) (width 0.2) (layer "F.Cu") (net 3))
 (segment (start 124.2061 106.26) (end 127.84 109.8939) (width 0.2) (layer "F.Cu") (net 3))
 (segment (start 179.6699 96.1068) (end 184.3 91.4767) (width 0.2) (layer "F.Cu") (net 3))
 (segment (start 121.72 96.2433) (end 121.72 94) (width 0.2) (layer "F.Cu") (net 3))
 (segment (start 183.374 113.28) (end 183.374 109.2493) (width 0.2) (layer "F.Cu") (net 3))
 (segment (start 135 111.7983) (end 127.84 111.7983) (width 0.2) (layer "F.Cu") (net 3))
 (segment (start 164.571 109.6706) (end 166.24 111.3396) (width 0.2) (layer "F.Cu") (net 3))
 (segment (start 121.7 97.74) (end 121.7 99.2167) (width 0.2) (layer "F.Cu") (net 3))
 (segment (start 183.374 113.28) (end 179 113.28) (width 0.2) (layer "F.Cu") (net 3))
 (segment (start 138 113) (end 139.4767 113) (width 0.2) (layer "F.Cu") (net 3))
 (segment (start 144 113) (end 139.4767 113) (width 0.2) (layer "F.Cu") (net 3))
 (segment (start 121.7 106.26) (end 121.7 99.2167) (width 0.2) (layer "F.Cu") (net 3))
 (segment (start 138 113) (end 136.5233 113) (width 0.2) (layer "F.Cu") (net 3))
 (segment (start 183.374 109.2493) (end 179.6699 105.5452) (width 0.2) (layer "F.Cu") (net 3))
 (segment (start 177.4967 113.28) (end 177.4767 113.3) (width 0.2) (layer "F.Cu") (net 3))
 (segment (start 127.84 114) (end 127.84 111.7983) (width 0.2) (layer "F.Cu") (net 3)))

